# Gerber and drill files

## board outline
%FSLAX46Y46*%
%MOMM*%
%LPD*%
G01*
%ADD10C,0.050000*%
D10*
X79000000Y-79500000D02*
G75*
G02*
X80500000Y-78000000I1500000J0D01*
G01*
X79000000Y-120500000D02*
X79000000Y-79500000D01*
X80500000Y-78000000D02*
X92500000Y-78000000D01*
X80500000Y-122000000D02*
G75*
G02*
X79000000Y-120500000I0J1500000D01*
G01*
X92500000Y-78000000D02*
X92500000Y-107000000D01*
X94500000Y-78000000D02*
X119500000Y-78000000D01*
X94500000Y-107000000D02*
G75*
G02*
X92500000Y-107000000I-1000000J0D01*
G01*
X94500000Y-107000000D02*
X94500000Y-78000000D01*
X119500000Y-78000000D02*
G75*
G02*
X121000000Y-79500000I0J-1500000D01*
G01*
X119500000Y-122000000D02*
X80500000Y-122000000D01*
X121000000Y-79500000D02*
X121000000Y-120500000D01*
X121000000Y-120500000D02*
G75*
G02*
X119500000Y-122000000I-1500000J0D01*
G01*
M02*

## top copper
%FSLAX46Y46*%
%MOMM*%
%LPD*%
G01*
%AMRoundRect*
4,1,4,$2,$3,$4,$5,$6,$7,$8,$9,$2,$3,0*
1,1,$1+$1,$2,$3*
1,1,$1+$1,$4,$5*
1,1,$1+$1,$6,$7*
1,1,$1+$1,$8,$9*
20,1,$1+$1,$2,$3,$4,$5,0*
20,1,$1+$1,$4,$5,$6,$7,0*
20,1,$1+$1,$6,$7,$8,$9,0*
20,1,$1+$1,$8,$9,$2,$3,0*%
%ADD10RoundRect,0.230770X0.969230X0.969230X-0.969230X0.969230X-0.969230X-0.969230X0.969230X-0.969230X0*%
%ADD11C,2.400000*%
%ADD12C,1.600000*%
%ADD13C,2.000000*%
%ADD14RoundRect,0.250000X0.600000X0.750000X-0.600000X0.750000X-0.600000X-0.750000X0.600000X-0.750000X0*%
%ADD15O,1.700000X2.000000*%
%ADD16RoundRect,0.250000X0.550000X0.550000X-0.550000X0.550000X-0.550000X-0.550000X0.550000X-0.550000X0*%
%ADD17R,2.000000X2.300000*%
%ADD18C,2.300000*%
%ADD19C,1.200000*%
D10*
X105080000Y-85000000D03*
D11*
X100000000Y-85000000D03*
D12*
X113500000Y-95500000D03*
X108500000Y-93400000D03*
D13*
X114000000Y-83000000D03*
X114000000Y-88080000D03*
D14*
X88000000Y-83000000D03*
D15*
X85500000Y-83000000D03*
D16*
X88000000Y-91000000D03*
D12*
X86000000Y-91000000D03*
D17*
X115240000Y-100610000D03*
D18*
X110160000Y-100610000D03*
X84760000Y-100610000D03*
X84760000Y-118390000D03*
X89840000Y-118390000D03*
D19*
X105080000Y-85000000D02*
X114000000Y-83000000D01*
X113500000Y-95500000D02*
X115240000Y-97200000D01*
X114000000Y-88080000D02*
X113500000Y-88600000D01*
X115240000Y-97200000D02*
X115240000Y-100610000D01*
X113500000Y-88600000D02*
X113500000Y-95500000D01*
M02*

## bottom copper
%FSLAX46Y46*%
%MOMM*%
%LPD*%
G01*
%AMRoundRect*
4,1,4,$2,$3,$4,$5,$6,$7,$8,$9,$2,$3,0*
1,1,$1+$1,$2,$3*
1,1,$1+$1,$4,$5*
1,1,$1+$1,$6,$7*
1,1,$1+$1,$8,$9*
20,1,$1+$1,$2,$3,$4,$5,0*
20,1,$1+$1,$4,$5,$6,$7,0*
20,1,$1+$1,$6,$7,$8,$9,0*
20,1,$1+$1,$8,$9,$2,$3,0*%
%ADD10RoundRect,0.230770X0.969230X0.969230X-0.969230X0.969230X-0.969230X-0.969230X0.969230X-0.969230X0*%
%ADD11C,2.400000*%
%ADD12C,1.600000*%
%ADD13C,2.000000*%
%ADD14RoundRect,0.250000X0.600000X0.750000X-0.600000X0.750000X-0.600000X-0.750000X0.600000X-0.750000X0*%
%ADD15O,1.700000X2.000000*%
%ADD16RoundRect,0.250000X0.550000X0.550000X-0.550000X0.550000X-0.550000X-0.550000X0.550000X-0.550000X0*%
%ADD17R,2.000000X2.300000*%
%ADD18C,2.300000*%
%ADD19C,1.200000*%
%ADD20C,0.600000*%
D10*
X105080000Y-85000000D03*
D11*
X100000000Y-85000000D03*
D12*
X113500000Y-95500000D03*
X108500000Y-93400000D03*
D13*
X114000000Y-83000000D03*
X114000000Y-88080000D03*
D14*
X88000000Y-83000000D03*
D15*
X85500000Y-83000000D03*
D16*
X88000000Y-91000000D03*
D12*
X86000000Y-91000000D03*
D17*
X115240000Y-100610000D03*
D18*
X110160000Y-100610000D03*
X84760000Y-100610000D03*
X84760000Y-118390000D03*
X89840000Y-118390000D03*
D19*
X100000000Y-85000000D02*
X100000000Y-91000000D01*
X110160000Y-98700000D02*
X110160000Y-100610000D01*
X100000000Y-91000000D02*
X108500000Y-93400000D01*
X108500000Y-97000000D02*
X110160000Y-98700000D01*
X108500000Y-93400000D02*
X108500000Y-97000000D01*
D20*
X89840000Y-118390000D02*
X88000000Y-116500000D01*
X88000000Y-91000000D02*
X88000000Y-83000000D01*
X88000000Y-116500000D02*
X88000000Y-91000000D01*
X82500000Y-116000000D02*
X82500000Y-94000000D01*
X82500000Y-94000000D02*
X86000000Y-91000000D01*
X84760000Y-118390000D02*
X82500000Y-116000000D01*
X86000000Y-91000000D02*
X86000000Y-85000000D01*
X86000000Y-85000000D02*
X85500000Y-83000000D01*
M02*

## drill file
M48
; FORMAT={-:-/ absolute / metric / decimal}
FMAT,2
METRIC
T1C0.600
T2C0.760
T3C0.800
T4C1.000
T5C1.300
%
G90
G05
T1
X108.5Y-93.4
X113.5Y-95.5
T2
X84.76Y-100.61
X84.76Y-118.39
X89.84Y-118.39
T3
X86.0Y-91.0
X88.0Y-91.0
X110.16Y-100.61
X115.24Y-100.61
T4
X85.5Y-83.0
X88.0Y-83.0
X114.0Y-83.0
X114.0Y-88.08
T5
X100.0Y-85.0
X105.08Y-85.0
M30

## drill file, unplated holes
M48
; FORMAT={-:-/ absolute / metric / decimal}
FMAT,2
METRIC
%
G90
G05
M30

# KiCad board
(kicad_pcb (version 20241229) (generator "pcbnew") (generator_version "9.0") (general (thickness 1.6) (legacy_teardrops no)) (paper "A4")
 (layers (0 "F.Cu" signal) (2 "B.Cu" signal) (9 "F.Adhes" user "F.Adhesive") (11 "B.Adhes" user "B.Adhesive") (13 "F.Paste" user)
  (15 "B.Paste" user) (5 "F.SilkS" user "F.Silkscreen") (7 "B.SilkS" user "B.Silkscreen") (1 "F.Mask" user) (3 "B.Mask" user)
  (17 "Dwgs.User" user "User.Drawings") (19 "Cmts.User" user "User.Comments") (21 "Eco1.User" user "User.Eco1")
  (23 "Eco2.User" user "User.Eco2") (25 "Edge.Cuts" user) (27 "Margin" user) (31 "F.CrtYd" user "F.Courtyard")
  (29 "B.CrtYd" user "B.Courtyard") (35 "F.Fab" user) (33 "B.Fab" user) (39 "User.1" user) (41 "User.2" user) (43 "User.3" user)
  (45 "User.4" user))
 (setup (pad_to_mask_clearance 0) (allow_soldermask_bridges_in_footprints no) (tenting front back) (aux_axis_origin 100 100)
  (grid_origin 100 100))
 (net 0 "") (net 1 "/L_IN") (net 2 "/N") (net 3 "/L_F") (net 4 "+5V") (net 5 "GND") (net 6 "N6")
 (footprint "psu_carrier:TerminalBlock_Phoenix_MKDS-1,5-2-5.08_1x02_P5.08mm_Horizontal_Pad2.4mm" (layer "F.Cu") (at 105.08 85 180)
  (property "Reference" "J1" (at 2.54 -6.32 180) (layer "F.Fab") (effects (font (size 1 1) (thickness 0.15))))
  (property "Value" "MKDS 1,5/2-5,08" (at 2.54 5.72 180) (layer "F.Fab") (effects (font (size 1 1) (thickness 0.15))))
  (pad "1" thru_hole roundrect (at 0 0 180) (size 2.4 2.4) (drill 1.3) (layers "*.Cu" "*.Mask") (remove_unused_layers no)
   (roundrect_rratio 0.096154) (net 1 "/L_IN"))
  (pad "2" thru_hole circle (at 5.08 0 180) (size 2.4 2.4) (drill 1.3) (layers "*.Cu" "*.Mask") (remove_unused_layers no) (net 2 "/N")))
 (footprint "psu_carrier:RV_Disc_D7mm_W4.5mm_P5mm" (layer "F.Cu") (at 113.5 95.5 180)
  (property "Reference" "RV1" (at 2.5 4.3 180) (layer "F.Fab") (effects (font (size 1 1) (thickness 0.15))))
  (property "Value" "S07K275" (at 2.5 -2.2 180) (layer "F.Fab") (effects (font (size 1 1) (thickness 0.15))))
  (pad "1" thru_hole circle (at 0 0 180) (size 1.6 1.6) (drill 0.6) (layers "*.Cu" "*.Mask") (remove_unused_layers no) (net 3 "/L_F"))
  (pad "2" thru_hole circle (at 5 2.1 180) (size 1.6 1.6) (drill 0.6) (layers "*.Cu" "*.Mask") (remove_unused_layers no) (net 2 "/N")))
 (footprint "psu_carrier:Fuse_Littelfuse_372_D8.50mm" (layer "F.Cu") (at 114 83 -90)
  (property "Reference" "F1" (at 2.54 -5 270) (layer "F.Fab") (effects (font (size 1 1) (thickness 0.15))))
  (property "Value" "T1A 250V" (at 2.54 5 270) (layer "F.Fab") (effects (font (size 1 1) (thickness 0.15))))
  (pad "1" thru_hole circle (at 0 0 270) (size 2 2) (drill 1) (layers "*.Cu" "*.Mask") (remove_unused_layers no) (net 1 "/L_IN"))
  (pad "2" thru_hole circle (at 5.08 0 270) (size 2 2) (drill 1) (layers "*.Cu" "*.Mask") (remove_unused_layers no) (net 3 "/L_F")))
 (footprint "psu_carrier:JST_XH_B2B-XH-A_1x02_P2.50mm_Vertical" (layer "F.Cu") (at 88 83 180)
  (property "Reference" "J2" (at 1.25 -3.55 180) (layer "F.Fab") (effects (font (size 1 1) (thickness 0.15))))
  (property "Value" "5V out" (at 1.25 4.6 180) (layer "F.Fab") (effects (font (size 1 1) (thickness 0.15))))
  (pad "1" thru_hole roundrect (at 0 0 180) (size 1.7 2) (drill 1) (layers "*.Cu" "*.Mask") (remove_unused_layers no)
   (roundrect_rratio 0.147059) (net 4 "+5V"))
  (pad "2" thru_hole oval (at 2.5 0 180) (size 1.7 2) (drill 1) (layers "*.Cu" "*.Mask") (remove_unused_layers no) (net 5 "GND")))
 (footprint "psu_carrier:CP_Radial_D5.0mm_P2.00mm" (layer "F.Cu") (at 88 91 180)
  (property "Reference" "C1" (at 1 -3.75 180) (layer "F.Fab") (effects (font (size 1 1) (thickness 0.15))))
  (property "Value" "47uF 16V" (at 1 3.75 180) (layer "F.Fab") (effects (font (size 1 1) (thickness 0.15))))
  (pad "1" thru_hole roundrect (at 0 0 180) (size 1.6 1.6) (drill 0.8) (layers "*.Cu" "*.Mask") (remove_unused_layers no)
   (roundrect_rratio 0.15625) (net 4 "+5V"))
  (pad "2" thru_hole circle (at 2 0 180) (size 1.6 1.6) (drill 0.8) (layers "*.Cu" "*.Mask") (remove_unused_layers no) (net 5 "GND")))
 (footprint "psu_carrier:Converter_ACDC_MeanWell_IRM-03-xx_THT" (layer "F.Cu") (at 115.24 100.61 -90)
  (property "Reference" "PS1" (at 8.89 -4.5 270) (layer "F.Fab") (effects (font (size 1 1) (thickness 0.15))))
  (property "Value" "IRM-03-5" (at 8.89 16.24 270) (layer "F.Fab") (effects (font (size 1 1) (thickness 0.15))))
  (pad "1" thru_hole rect (at 0 0 270) (size 2.3 2) (drill 0.8) (layers "*.Cu" "*.Mask") (remove_unused_layers no) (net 3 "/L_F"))
  (pad "3" thru_hole circle (at 0 5.08 270) (size 2.3 2.3) (drill 0.8) (layers "*.Cu" "*.Mask") (remove_unused_layers no) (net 2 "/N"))
  (pad "5" thru_hole circle (at 0 30.48 270) (size 2.3 2.3) (drill 0.76) (layers "*.Cu" "*.Mask") (remove_unused_layers no) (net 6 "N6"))
  (pad "14" thru_hole circle (at 17.78 30.48 270) (size 2.3 2.3) (drill 0.76) (layers "*.Cu" "*.Mask") (remove_unused_layers no)
   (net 5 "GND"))
  (pad "16" thru_hole circle (at 17.78 25.4 270) (size 2.3 2.3) (drill 0.76) (layers "*.Cu" "*.Mask") (remove_unused_layers no)
   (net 4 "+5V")))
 (gr_arc (start 79 79.5) (mid 79.439339 78.439339) (end 80.5 78) (stroke (width 0.05) (type default)) (layer "Edge.Cuts"))
 (gr_line (start 79 120.5) (end 79 79.5) (stroke (width 0.05) (type default)) (layer "Edge.Cuts"))
 (gr_line (start 80.5 78) (end 92.5 78) (stroke (width 0.05) (type default)) (layer "Edge.Cuts"))
 (gr_arc (start 80.5 122) (mid 79.439339 121.56066) (end 79 120.5) (stroke (width 0.05) (type default)) (layer "Edge.Cuts"))
 (gr_line (start 92.5 78) (end 92.5 107) (stroke (width 0.05) (type default)) (layer "Edge.Cuts"))
 (gr_line (start 94.5 78) (end 119.5 78) (stroke (width 0.05) (type default)) (layer "Edge.Cuts"))
 (gr_arc (start 94.5 107) (mid 93.5 108) (end 92.5 107) (stroke (width 0.05) (type default)) (layer "Edge.Cuts"))
 (gr_line (start 94.5 107) (end 94.5 78) (stroke (width 0.05) (type default)) (layer "Edge.Cuts"))
 (gr_arc (start 119.5 78) (mid 120.56066 78.439339) (end 121 79.5) (stroke (width 0.05) (type default)) (layer "Edge.Cuts"))
 (gr_line (start 119.5 122) (end 80.5 122) (stroke (width 0.05) (type default)) (layer "Edge.Cuts"))
 (gr_line (start 121 79.5) (end 121 120.5) (stroke (width 0.05) (type default)) (layer "Edge.Cuts"))
 (gr_arc (start 121 120.5) (mid 120.56066 121.56066) (end 119.5 122) (stroke (width 0.05) (type default)) (layer "Edge.Cuts"))
 (segment (start 105.08 85) (end 114 83) (width 1.2) (layer "F.Cu") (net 1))
 (segment (start 113.5 95.5) (end 115.24 97.2) (width 1.2) (layer "F.Cu") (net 3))
 (segment (start 114 88.08) (end 113.5 88.6) (width 1.2) (layer "F.Cu") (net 3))
 (segment (start 115.24 97.2) (end 115.24 100.61) (width 1.2) (layer "F.Cu") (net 3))
 (segment (start 113.5 88.6) (end 113.5 95.5) (width 1.2) (layer "F.Cu") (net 3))
 (segment (start 100 85) (end 100 91) (width 1.2) (layer "B.Cu") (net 2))
 (segment (start 110.16 98.7) (end 110.16 100.61) (width 1.2) (layer "B.Cu") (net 2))
 (segment (start 100 91) (end 108.5 93.4) (width 1.2) (layer "B.Cu") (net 2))
 (segment (start 108.5 97) (end 110.16 98.7) (width 1.2) (layer "B.Cu") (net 2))
 (segment (start 108.5 93.4) (end 108.5 97) (width 1.2) (layer "B.Cu") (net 2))
 (segment (start 89.84 118.39) (end 88 116.5) (width 0.6) (layer "B.Cu") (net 4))
 (segment (start 88 91) (end 88 83) (width 0.6) (layer "B.Cu") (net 4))
 (segment (start 88 116.5) (end 88 91) (width 0.6) (layer "B.Cu") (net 4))
 (segment (start 82.5 116) (end 82.5 94) (width 0.6) (layer "B.Cu") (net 5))
 (segment (start 82.5 94) (end 86 91) (width 0.6) (layer "B.Cu") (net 5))
 (segment (start 84.76 118.39) (end 82.5 116) (width 0.6) (layer "B.Cu") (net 5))
 (segment (start 86 91) (end 86 85) (width 0.6) (layer "B.Cu") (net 5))
 (segment (start 86 85) (end 85.5 83) (width 0.6) (layer "B.Cu") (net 5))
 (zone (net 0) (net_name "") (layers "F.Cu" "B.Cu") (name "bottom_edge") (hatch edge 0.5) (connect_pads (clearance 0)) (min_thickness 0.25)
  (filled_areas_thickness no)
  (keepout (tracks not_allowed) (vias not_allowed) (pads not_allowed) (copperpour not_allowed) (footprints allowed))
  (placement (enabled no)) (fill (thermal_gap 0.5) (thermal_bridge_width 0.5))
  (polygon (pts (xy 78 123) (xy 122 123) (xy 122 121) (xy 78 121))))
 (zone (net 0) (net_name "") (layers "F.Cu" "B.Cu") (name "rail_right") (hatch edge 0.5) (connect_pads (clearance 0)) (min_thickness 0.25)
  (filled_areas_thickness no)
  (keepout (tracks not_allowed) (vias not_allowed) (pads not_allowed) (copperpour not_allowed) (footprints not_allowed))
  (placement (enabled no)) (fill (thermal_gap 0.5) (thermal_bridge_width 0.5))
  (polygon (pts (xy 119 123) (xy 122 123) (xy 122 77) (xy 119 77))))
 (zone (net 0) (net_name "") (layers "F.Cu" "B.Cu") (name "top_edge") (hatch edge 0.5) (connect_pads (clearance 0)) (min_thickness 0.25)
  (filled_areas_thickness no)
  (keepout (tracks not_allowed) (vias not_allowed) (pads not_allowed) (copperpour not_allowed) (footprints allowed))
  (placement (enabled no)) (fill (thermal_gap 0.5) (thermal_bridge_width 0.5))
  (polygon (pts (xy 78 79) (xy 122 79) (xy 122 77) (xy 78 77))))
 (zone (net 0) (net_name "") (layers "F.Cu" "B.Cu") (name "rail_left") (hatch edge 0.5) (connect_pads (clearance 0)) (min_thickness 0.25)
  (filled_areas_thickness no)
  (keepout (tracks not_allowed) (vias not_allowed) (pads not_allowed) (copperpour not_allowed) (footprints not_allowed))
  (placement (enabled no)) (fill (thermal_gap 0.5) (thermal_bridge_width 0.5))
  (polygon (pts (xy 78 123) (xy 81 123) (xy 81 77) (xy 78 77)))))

